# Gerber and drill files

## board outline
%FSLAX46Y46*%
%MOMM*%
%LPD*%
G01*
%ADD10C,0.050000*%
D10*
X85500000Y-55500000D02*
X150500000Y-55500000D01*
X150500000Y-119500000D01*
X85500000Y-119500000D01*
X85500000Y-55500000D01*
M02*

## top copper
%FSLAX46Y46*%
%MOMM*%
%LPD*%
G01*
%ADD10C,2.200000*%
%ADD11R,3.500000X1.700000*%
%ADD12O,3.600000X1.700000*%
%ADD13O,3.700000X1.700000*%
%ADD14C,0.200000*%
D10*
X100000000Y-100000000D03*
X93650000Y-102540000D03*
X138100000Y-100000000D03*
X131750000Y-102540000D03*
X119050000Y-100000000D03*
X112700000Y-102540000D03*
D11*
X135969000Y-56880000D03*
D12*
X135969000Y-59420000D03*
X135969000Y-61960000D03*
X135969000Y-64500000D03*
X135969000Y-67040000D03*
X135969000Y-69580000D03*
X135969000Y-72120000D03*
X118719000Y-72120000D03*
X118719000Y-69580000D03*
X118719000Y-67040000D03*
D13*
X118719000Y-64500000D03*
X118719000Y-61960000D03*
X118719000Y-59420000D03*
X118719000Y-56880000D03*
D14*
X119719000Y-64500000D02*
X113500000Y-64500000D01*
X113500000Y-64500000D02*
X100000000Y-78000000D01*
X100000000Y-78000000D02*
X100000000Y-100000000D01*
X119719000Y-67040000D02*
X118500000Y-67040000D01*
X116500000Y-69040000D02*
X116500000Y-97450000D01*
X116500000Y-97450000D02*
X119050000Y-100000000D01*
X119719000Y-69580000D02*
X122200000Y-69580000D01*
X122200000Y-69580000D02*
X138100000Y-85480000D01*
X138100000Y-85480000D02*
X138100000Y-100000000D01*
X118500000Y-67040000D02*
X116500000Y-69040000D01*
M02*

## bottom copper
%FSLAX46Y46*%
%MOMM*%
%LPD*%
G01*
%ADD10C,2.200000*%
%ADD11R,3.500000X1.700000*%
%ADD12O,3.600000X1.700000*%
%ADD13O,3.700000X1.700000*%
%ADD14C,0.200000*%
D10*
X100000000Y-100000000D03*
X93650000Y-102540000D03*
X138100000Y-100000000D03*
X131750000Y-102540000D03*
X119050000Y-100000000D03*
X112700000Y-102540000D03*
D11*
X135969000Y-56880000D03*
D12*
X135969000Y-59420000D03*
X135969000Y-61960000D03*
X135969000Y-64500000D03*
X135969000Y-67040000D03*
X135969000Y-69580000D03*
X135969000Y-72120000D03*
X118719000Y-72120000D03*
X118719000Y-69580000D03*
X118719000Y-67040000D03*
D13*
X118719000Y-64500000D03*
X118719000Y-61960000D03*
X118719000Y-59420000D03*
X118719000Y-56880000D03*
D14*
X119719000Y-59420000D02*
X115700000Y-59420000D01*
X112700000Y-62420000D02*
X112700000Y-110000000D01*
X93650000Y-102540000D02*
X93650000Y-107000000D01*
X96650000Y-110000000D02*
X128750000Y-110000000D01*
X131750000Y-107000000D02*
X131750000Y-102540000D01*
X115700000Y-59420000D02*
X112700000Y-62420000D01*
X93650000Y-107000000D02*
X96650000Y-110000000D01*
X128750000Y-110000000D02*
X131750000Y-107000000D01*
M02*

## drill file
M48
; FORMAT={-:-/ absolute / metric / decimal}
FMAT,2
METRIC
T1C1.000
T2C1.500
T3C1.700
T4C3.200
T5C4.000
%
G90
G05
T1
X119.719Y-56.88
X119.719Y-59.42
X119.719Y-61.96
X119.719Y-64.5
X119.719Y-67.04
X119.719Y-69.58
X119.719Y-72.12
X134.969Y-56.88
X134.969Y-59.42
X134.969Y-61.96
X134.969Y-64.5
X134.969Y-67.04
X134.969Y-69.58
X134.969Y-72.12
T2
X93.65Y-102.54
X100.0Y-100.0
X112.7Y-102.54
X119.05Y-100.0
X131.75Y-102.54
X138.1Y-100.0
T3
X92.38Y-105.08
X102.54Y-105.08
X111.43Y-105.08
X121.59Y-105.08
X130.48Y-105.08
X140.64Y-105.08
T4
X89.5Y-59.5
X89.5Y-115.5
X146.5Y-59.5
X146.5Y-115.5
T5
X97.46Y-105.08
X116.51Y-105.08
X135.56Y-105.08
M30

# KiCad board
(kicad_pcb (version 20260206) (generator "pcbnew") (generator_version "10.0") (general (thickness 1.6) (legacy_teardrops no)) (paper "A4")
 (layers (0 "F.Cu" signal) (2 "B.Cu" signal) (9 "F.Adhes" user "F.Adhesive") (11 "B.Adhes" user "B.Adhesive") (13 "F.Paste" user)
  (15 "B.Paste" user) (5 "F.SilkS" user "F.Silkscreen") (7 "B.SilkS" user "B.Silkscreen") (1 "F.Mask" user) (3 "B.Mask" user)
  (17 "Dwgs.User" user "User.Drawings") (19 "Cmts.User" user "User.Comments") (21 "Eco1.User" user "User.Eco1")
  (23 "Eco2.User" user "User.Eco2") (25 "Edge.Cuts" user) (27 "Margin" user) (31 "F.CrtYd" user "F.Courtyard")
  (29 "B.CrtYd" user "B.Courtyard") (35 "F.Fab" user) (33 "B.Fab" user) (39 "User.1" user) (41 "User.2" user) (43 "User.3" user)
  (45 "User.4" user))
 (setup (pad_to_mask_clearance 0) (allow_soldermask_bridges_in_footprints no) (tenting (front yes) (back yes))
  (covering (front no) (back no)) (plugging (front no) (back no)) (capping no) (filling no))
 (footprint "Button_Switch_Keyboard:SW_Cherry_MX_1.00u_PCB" (layer "F.Cu") (at 100 100)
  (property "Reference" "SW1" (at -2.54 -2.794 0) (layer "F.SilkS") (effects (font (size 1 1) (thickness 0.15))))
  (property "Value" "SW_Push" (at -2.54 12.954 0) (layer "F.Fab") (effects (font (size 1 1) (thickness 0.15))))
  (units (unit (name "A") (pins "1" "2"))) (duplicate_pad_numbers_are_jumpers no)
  (pad "" np_thru_hole circle (at -7.62 5.08) (size 1.7 1.7) (drill 1.7) (layers "*.Cu" "*.Mask"))
  (pad "" np_thru_hole circle (at -2.54 5.08) (size 4 4) (drill 4) (layers "*.Cu" "*.Mask"))
  (pad "" np_thru_hole circle (at 2.54 5.08) (size 1.7 1.7) (drill 1.7) (layers "*.Cu" "*.Mask"))
  (pad "1" thru_hole circle (at 0 0) (size 2.2 2.2) (drill 1.5) (layers "*.Cu" "*.Mask") (remove_unused_layers no)
   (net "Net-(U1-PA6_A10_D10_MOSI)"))
  (pad "2" thru_hole circle (at -6.35 2.54) (size 2.2 2.2) (drill 1.5) (layers "*.Cu" "*.Mask") (remove_unused_layers no) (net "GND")))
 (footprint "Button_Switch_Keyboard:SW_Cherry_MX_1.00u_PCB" (layer "F.Cu") (at 138.1 100)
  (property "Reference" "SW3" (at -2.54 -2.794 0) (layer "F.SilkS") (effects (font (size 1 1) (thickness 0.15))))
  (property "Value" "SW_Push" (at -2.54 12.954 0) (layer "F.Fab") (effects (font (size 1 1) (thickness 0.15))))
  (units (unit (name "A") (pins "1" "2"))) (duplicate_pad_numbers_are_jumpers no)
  (pad "" np_thru_hole circle (at -7.62 5.08) (size 1.7 1.7) (drill 1.7) (layers "*.Cu" "*.Mask"))
  (pad "" np_thru_hole circle (at -2.54 5.08) (size 4 4) (drill 4) (layers "*.Cu" "*.Mask"))
  (pad "" np_thru_hole circle (at 2.54 5.08) (size 1.7 1.7) (drill 1.7) (layers "*.Cu" "*.Mask"))
  (pad "1" thru_hole circle (at 0 0) (size 2.2 2.2) (drill 1.5) (layers "*.Cu" "*.Mask") (remove_unused_layers no)
   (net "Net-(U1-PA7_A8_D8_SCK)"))
  (pad "2" thru_hole circle (at -6.35 2.54) (size 2.2 2.2) (drill 1.5) (layers "*.Cu" "*.Mask") (remove_unused_layers no) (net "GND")))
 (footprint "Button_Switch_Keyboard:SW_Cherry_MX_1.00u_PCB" (layer "F.Cu") (at 119.05 100)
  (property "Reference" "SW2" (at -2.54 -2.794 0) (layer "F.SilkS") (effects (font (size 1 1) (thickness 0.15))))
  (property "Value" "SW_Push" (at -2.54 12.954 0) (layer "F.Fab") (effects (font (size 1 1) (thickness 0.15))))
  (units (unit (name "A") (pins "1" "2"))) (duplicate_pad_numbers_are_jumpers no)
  (pad "" np_thru_hole circle (at -7.62 5.08) (size 1.7 1.7) (drill 1.7) (layers "*.Cu" "*.Mask"))
  (pad "" np_thru_hole circle (at -2.54 5.08) (size 4 4) (drill 4) (layers "*.Cu" "*.Mask"))
  (pad "" np_thru_hole circle (at 2.54 5.08) (size 1.7 1.7) (drill 1.7) (layers "*.Cu" "*.Mask"))
  (pad "1" thru_hole circle (at 0 0) (size 2.2 2.2) (drill 1.5) (layers "*.Cu" "*.Mask") (remove_unused_layers no)
   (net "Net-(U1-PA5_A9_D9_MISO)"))
  (pad "2" thru_hole circle (at -6.35 2.54) (size 2.2 2.2) (drill 1.5) (layers "*.Cu" "*.Mask") (remove_unused_layers no) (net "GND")))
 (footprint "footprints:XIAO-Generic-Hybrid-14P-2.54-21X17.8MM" (layer "B.Cu") (at 127.344 64.5 180)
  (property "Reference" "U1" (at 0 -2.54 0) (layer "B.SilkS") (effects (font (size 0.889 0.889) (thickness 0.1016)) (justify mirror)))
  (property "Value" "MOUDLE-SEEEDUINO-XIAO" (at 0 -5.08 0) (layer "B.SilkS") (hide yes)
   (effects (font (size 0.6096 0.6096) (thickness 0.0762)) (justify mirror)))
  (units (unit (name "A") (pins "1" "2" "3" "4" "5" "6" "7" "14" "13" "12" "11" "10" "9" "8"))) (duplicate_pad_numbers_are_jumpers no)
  (pad "1" thru_hole rect (at -7.625 7.62 180) (size 3.5 1.7) (drill 1 (offset -1 0)) (layers "*.Cu" "*.Mask") (remove_unused_layers no)
   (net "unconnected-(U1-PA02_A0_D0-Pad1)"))
  (pad "2" thru_hole oval (at -7.625 5.08 180) (size 3.6 1.7) (drill 1 (offset -1 0)) (layers "*.Cu" "*.Mask") (remove_unused_layers no)
   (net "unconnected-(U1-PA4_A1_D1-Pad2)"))
  (pad "3" thru_hole oval (at -7.625 2.54 180) (size 3.6 1.7) (drill 1 (offset -1 0)) (layers "*.Cu" "*.Mask") (remove_unused_layers no)
   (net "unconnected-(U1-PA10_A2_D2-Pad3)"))
  (pad "4" thru_hole oval (at -7.625 0 180) (size 3.6 1.7) (drill 1 (offset -1 0)) (layers "*.Cu" "*.Mask") (remove_unused_layers no)
   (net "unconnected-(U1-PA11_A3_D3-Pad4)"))
  (pad "5" thru_hole oval (at -7.625 -2.54 180) (size 3.6 1.7) (drill 1 (offset -1 0)) (layers "*.Cu" "*.Mask") (remove_unused_layers no)
   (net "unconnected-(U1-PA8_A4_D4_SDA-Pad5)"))
  (pad "6" thru_hole oval (at -7.625 -5.08) (size 3.6 1.7) (drill 1 (offset 1 0)) (layers "*.Cu" "*.Mask") (remove_unused_layers no)
   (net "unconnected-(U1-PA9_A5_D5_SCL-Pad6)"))
  (pad "7" thru_hole oval (at -7.625 -7.62 180) (size 3.6 1.7) (drill 1 (offset -1 0)) (layers "*.Cu" "*.Mask") (remove_unused_layers no)
   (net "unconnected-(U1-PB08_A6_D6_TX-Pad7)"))
  (pad "8" thru_hole oval (at 7.625 -7.62 180) (size 3.6 1.7) (drill 1 (offset 1 0)) (layers "*.Cu" "*.Mask") (remove_unused_layers no)
   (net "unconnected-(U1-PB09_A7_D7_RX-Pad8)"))
  (pad "9" thru_hole oval (at 7.625 -5.08 180) (size 3.6 1.7) (drill 1 (offset 1 0)) (layers "*.Cu" "*.Mask") (remove_unused_layers no)
   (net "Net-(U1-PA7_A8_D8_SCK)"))
  (pad "10" thru_hole oval (at 7.625 -2.54 180) (size 3.6 1.7) (drill 1 (offset 1 0)) (layers "*.Cu" "*.Mask") (remove_unused_layers no)
   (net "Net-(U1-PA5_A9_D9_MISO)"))
  (pad "11" thru_hole oval (at 7.625 0 180) (size 3.7 1.7) (drill 1 (offset 1 0)) (layers "*.Cu" "*.Mask") (remove_unused_layers no)
   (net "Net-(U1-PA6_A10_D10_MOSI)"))
  (pad "12" thru_hole oval (at 7.625 2.54 180) (size 3.7 1.7) (drill 1 (offset 1 0)) (layers "*.Cu" "*.Mask") (remove_unused_layers no)
   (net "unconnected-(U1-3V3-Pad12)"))
  (pad "13" thru_hole oval (at 7.625 5.08 180) (size 3.7 1.7) (drill 1 (offset 1 0)) (layers "*.Cu" "*.Mask") (remove_unused_layers no)
   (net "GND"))
  (pad "14" thru_hole oval (at 7.625 7.62 180) (size 3.7 1.7) (drill 1 (offset 1 0)) (layers "*.Cu" "*.Mask") (remove_unused_layers no)
   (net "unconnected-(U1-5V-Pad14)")))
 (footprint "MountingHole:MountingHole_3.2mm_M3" (layer "F.Cu") (at 89.5 59.5)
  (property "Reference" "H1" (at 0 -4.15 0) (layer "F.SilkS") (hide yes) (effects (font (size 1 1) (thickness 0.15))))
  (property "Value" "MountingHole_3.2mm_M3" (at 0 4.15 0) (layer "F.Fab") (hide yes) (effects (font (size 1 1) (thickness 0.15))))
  (pad "" np_thru_hole circle (at 0 0) (size 3.2 3.2) (drill 3.2) (layers "*.Cu" "*.Mask")))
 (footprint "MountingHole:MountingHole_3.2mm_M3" (layer "F.Cu") (at 146.5 59.5)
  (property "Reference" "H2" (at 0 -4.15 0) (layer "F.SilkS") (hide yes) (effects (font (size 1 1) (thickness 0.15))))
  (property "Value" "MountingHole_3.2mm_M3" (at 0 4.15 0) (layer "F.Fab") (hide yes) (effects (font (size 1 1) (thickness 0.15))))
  (pad "" np_thru_hole circle (at 0 0) (size 3.2 3.2) (drill 3.2) (layers "*.Cu" "*.Mask")))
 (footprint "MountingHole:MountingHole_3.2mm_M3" (layer "F.Cu") (at 89.5 115.5)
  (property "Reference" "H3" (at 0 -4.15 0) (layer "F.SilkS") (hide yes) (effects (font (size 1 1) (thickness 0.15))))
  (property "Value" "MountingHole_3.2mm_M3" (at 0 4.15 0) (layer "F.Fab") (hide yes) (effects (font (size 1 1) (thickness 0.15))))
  (pad "" np_thru_hole circle (at 0 0) (size 3.2 3.2) (drill 3.2) (layers "*.Cu" "*.Mask")))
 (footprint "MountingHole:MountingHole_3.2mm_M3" (layer "F.Cu") (at 146.5 115.5)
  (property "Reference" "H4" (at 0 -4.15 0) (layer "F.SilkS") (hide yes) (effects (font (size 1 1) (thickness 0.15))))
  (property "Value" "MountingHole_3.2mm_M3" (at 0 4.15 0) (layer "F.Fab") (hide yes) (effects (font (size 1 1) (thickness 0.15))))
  (pad "" np_thru_hole circle (at 0 0) (size 3.2 3.2) (drill 3.2) (layers "*.Cu" "*.Mask")))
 (gr_rect (start 85.5 55.5) (end 150.5 119.5) (stroke (width 0.05) (type default)) (fill no) (layer "Edge.Cuts"))
 (segment (start 119.71900 64.50000) (end 113.50000 64.50000) (width 0.2) (layer "F.Cu") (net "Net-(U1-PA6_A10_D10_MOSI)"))
 (segment (start 113.50000 64.50000) (end 100.00000 78.00000) (width 0.2) (layer "F.Cu") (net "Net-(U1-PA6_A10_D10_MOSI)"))
 (segment (start 100.00000 78.00000) (end 100.00000 100.00000) (width 0.2) (layer "F.Cu") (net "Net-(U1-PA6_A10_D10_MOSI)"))
 (segment (start 119.71900 67.04000) (end 118.50000 67.04000) (width 0.2) (layer "F.Cu") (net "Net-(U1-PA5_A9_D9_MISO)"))
 (segment (start 116.50000 69.04000) (end 116.50000 97.45000) (width 0.2) (layer "F.Cu") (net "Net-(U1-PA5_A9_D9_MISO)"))
 (segment (start 116.50000 97.45000) (end 119.05000 100.00000) (width 0.2) (layer "F.Cu") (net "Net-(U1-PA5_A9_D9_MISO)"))
 (segment (start 119.71900 69.58000) (end 122.20000 69.58000) (width 0.2) (layer "F.Cu") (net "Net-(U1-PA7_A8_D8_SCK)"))
 (segment (start 122.20000 69.58000) (end 138.10000 85.48000) (width 0.2) (layer "F.Cu") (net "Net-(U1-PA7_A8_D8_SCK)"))
 (segment (start 138.10000 85.48000) (end 138.10000 100.00000) (width 0.2) (layer "F.Cu") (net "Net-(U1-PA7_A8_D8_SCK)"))
 (segment (start 119.71900 59.42000) (end 115.70000 59.42000) (width 0.2) (layer "B.Cu") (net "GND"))
 (segment (start 112.70000 62.42000) (end 112.70000 110.00000) (width 0.2) (layer "B.Cu") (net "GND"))
 (segment (start 93.65000 102.54000) (end 93.65000 107.00000) (width 0.2) (layer "B.Cu") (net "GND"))
 (segment (start 96.65000 110.00000) (end 128.75000 110.00000) (width 0.2) (layer "B.Cu") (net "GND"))
 (segment (start 131.75000 107.00000) (end 131.75000 102.54000) (width 0.2) (layer "B.Cu") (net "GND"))
 (segment (start 118.50000 67.04000) (end 116.50000 69.04000) (width 0.2) (layer "F.Cu") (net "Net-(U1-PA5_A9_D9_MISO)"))
 (segment (start 115.70000 59.42000) (end 112.70000 62.42000) (width 0.2) (layer "B.Cu") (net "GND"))
 (segment (start 93.65000 107.00000) (end 96.65000 110.00000) (width 0.2) (layer "B.Cu") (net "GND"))
 (segment (start 128.75000 110.00000) (end 131.75000 107.00000) (width 0.2) (layer "B.Cu") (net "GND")))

